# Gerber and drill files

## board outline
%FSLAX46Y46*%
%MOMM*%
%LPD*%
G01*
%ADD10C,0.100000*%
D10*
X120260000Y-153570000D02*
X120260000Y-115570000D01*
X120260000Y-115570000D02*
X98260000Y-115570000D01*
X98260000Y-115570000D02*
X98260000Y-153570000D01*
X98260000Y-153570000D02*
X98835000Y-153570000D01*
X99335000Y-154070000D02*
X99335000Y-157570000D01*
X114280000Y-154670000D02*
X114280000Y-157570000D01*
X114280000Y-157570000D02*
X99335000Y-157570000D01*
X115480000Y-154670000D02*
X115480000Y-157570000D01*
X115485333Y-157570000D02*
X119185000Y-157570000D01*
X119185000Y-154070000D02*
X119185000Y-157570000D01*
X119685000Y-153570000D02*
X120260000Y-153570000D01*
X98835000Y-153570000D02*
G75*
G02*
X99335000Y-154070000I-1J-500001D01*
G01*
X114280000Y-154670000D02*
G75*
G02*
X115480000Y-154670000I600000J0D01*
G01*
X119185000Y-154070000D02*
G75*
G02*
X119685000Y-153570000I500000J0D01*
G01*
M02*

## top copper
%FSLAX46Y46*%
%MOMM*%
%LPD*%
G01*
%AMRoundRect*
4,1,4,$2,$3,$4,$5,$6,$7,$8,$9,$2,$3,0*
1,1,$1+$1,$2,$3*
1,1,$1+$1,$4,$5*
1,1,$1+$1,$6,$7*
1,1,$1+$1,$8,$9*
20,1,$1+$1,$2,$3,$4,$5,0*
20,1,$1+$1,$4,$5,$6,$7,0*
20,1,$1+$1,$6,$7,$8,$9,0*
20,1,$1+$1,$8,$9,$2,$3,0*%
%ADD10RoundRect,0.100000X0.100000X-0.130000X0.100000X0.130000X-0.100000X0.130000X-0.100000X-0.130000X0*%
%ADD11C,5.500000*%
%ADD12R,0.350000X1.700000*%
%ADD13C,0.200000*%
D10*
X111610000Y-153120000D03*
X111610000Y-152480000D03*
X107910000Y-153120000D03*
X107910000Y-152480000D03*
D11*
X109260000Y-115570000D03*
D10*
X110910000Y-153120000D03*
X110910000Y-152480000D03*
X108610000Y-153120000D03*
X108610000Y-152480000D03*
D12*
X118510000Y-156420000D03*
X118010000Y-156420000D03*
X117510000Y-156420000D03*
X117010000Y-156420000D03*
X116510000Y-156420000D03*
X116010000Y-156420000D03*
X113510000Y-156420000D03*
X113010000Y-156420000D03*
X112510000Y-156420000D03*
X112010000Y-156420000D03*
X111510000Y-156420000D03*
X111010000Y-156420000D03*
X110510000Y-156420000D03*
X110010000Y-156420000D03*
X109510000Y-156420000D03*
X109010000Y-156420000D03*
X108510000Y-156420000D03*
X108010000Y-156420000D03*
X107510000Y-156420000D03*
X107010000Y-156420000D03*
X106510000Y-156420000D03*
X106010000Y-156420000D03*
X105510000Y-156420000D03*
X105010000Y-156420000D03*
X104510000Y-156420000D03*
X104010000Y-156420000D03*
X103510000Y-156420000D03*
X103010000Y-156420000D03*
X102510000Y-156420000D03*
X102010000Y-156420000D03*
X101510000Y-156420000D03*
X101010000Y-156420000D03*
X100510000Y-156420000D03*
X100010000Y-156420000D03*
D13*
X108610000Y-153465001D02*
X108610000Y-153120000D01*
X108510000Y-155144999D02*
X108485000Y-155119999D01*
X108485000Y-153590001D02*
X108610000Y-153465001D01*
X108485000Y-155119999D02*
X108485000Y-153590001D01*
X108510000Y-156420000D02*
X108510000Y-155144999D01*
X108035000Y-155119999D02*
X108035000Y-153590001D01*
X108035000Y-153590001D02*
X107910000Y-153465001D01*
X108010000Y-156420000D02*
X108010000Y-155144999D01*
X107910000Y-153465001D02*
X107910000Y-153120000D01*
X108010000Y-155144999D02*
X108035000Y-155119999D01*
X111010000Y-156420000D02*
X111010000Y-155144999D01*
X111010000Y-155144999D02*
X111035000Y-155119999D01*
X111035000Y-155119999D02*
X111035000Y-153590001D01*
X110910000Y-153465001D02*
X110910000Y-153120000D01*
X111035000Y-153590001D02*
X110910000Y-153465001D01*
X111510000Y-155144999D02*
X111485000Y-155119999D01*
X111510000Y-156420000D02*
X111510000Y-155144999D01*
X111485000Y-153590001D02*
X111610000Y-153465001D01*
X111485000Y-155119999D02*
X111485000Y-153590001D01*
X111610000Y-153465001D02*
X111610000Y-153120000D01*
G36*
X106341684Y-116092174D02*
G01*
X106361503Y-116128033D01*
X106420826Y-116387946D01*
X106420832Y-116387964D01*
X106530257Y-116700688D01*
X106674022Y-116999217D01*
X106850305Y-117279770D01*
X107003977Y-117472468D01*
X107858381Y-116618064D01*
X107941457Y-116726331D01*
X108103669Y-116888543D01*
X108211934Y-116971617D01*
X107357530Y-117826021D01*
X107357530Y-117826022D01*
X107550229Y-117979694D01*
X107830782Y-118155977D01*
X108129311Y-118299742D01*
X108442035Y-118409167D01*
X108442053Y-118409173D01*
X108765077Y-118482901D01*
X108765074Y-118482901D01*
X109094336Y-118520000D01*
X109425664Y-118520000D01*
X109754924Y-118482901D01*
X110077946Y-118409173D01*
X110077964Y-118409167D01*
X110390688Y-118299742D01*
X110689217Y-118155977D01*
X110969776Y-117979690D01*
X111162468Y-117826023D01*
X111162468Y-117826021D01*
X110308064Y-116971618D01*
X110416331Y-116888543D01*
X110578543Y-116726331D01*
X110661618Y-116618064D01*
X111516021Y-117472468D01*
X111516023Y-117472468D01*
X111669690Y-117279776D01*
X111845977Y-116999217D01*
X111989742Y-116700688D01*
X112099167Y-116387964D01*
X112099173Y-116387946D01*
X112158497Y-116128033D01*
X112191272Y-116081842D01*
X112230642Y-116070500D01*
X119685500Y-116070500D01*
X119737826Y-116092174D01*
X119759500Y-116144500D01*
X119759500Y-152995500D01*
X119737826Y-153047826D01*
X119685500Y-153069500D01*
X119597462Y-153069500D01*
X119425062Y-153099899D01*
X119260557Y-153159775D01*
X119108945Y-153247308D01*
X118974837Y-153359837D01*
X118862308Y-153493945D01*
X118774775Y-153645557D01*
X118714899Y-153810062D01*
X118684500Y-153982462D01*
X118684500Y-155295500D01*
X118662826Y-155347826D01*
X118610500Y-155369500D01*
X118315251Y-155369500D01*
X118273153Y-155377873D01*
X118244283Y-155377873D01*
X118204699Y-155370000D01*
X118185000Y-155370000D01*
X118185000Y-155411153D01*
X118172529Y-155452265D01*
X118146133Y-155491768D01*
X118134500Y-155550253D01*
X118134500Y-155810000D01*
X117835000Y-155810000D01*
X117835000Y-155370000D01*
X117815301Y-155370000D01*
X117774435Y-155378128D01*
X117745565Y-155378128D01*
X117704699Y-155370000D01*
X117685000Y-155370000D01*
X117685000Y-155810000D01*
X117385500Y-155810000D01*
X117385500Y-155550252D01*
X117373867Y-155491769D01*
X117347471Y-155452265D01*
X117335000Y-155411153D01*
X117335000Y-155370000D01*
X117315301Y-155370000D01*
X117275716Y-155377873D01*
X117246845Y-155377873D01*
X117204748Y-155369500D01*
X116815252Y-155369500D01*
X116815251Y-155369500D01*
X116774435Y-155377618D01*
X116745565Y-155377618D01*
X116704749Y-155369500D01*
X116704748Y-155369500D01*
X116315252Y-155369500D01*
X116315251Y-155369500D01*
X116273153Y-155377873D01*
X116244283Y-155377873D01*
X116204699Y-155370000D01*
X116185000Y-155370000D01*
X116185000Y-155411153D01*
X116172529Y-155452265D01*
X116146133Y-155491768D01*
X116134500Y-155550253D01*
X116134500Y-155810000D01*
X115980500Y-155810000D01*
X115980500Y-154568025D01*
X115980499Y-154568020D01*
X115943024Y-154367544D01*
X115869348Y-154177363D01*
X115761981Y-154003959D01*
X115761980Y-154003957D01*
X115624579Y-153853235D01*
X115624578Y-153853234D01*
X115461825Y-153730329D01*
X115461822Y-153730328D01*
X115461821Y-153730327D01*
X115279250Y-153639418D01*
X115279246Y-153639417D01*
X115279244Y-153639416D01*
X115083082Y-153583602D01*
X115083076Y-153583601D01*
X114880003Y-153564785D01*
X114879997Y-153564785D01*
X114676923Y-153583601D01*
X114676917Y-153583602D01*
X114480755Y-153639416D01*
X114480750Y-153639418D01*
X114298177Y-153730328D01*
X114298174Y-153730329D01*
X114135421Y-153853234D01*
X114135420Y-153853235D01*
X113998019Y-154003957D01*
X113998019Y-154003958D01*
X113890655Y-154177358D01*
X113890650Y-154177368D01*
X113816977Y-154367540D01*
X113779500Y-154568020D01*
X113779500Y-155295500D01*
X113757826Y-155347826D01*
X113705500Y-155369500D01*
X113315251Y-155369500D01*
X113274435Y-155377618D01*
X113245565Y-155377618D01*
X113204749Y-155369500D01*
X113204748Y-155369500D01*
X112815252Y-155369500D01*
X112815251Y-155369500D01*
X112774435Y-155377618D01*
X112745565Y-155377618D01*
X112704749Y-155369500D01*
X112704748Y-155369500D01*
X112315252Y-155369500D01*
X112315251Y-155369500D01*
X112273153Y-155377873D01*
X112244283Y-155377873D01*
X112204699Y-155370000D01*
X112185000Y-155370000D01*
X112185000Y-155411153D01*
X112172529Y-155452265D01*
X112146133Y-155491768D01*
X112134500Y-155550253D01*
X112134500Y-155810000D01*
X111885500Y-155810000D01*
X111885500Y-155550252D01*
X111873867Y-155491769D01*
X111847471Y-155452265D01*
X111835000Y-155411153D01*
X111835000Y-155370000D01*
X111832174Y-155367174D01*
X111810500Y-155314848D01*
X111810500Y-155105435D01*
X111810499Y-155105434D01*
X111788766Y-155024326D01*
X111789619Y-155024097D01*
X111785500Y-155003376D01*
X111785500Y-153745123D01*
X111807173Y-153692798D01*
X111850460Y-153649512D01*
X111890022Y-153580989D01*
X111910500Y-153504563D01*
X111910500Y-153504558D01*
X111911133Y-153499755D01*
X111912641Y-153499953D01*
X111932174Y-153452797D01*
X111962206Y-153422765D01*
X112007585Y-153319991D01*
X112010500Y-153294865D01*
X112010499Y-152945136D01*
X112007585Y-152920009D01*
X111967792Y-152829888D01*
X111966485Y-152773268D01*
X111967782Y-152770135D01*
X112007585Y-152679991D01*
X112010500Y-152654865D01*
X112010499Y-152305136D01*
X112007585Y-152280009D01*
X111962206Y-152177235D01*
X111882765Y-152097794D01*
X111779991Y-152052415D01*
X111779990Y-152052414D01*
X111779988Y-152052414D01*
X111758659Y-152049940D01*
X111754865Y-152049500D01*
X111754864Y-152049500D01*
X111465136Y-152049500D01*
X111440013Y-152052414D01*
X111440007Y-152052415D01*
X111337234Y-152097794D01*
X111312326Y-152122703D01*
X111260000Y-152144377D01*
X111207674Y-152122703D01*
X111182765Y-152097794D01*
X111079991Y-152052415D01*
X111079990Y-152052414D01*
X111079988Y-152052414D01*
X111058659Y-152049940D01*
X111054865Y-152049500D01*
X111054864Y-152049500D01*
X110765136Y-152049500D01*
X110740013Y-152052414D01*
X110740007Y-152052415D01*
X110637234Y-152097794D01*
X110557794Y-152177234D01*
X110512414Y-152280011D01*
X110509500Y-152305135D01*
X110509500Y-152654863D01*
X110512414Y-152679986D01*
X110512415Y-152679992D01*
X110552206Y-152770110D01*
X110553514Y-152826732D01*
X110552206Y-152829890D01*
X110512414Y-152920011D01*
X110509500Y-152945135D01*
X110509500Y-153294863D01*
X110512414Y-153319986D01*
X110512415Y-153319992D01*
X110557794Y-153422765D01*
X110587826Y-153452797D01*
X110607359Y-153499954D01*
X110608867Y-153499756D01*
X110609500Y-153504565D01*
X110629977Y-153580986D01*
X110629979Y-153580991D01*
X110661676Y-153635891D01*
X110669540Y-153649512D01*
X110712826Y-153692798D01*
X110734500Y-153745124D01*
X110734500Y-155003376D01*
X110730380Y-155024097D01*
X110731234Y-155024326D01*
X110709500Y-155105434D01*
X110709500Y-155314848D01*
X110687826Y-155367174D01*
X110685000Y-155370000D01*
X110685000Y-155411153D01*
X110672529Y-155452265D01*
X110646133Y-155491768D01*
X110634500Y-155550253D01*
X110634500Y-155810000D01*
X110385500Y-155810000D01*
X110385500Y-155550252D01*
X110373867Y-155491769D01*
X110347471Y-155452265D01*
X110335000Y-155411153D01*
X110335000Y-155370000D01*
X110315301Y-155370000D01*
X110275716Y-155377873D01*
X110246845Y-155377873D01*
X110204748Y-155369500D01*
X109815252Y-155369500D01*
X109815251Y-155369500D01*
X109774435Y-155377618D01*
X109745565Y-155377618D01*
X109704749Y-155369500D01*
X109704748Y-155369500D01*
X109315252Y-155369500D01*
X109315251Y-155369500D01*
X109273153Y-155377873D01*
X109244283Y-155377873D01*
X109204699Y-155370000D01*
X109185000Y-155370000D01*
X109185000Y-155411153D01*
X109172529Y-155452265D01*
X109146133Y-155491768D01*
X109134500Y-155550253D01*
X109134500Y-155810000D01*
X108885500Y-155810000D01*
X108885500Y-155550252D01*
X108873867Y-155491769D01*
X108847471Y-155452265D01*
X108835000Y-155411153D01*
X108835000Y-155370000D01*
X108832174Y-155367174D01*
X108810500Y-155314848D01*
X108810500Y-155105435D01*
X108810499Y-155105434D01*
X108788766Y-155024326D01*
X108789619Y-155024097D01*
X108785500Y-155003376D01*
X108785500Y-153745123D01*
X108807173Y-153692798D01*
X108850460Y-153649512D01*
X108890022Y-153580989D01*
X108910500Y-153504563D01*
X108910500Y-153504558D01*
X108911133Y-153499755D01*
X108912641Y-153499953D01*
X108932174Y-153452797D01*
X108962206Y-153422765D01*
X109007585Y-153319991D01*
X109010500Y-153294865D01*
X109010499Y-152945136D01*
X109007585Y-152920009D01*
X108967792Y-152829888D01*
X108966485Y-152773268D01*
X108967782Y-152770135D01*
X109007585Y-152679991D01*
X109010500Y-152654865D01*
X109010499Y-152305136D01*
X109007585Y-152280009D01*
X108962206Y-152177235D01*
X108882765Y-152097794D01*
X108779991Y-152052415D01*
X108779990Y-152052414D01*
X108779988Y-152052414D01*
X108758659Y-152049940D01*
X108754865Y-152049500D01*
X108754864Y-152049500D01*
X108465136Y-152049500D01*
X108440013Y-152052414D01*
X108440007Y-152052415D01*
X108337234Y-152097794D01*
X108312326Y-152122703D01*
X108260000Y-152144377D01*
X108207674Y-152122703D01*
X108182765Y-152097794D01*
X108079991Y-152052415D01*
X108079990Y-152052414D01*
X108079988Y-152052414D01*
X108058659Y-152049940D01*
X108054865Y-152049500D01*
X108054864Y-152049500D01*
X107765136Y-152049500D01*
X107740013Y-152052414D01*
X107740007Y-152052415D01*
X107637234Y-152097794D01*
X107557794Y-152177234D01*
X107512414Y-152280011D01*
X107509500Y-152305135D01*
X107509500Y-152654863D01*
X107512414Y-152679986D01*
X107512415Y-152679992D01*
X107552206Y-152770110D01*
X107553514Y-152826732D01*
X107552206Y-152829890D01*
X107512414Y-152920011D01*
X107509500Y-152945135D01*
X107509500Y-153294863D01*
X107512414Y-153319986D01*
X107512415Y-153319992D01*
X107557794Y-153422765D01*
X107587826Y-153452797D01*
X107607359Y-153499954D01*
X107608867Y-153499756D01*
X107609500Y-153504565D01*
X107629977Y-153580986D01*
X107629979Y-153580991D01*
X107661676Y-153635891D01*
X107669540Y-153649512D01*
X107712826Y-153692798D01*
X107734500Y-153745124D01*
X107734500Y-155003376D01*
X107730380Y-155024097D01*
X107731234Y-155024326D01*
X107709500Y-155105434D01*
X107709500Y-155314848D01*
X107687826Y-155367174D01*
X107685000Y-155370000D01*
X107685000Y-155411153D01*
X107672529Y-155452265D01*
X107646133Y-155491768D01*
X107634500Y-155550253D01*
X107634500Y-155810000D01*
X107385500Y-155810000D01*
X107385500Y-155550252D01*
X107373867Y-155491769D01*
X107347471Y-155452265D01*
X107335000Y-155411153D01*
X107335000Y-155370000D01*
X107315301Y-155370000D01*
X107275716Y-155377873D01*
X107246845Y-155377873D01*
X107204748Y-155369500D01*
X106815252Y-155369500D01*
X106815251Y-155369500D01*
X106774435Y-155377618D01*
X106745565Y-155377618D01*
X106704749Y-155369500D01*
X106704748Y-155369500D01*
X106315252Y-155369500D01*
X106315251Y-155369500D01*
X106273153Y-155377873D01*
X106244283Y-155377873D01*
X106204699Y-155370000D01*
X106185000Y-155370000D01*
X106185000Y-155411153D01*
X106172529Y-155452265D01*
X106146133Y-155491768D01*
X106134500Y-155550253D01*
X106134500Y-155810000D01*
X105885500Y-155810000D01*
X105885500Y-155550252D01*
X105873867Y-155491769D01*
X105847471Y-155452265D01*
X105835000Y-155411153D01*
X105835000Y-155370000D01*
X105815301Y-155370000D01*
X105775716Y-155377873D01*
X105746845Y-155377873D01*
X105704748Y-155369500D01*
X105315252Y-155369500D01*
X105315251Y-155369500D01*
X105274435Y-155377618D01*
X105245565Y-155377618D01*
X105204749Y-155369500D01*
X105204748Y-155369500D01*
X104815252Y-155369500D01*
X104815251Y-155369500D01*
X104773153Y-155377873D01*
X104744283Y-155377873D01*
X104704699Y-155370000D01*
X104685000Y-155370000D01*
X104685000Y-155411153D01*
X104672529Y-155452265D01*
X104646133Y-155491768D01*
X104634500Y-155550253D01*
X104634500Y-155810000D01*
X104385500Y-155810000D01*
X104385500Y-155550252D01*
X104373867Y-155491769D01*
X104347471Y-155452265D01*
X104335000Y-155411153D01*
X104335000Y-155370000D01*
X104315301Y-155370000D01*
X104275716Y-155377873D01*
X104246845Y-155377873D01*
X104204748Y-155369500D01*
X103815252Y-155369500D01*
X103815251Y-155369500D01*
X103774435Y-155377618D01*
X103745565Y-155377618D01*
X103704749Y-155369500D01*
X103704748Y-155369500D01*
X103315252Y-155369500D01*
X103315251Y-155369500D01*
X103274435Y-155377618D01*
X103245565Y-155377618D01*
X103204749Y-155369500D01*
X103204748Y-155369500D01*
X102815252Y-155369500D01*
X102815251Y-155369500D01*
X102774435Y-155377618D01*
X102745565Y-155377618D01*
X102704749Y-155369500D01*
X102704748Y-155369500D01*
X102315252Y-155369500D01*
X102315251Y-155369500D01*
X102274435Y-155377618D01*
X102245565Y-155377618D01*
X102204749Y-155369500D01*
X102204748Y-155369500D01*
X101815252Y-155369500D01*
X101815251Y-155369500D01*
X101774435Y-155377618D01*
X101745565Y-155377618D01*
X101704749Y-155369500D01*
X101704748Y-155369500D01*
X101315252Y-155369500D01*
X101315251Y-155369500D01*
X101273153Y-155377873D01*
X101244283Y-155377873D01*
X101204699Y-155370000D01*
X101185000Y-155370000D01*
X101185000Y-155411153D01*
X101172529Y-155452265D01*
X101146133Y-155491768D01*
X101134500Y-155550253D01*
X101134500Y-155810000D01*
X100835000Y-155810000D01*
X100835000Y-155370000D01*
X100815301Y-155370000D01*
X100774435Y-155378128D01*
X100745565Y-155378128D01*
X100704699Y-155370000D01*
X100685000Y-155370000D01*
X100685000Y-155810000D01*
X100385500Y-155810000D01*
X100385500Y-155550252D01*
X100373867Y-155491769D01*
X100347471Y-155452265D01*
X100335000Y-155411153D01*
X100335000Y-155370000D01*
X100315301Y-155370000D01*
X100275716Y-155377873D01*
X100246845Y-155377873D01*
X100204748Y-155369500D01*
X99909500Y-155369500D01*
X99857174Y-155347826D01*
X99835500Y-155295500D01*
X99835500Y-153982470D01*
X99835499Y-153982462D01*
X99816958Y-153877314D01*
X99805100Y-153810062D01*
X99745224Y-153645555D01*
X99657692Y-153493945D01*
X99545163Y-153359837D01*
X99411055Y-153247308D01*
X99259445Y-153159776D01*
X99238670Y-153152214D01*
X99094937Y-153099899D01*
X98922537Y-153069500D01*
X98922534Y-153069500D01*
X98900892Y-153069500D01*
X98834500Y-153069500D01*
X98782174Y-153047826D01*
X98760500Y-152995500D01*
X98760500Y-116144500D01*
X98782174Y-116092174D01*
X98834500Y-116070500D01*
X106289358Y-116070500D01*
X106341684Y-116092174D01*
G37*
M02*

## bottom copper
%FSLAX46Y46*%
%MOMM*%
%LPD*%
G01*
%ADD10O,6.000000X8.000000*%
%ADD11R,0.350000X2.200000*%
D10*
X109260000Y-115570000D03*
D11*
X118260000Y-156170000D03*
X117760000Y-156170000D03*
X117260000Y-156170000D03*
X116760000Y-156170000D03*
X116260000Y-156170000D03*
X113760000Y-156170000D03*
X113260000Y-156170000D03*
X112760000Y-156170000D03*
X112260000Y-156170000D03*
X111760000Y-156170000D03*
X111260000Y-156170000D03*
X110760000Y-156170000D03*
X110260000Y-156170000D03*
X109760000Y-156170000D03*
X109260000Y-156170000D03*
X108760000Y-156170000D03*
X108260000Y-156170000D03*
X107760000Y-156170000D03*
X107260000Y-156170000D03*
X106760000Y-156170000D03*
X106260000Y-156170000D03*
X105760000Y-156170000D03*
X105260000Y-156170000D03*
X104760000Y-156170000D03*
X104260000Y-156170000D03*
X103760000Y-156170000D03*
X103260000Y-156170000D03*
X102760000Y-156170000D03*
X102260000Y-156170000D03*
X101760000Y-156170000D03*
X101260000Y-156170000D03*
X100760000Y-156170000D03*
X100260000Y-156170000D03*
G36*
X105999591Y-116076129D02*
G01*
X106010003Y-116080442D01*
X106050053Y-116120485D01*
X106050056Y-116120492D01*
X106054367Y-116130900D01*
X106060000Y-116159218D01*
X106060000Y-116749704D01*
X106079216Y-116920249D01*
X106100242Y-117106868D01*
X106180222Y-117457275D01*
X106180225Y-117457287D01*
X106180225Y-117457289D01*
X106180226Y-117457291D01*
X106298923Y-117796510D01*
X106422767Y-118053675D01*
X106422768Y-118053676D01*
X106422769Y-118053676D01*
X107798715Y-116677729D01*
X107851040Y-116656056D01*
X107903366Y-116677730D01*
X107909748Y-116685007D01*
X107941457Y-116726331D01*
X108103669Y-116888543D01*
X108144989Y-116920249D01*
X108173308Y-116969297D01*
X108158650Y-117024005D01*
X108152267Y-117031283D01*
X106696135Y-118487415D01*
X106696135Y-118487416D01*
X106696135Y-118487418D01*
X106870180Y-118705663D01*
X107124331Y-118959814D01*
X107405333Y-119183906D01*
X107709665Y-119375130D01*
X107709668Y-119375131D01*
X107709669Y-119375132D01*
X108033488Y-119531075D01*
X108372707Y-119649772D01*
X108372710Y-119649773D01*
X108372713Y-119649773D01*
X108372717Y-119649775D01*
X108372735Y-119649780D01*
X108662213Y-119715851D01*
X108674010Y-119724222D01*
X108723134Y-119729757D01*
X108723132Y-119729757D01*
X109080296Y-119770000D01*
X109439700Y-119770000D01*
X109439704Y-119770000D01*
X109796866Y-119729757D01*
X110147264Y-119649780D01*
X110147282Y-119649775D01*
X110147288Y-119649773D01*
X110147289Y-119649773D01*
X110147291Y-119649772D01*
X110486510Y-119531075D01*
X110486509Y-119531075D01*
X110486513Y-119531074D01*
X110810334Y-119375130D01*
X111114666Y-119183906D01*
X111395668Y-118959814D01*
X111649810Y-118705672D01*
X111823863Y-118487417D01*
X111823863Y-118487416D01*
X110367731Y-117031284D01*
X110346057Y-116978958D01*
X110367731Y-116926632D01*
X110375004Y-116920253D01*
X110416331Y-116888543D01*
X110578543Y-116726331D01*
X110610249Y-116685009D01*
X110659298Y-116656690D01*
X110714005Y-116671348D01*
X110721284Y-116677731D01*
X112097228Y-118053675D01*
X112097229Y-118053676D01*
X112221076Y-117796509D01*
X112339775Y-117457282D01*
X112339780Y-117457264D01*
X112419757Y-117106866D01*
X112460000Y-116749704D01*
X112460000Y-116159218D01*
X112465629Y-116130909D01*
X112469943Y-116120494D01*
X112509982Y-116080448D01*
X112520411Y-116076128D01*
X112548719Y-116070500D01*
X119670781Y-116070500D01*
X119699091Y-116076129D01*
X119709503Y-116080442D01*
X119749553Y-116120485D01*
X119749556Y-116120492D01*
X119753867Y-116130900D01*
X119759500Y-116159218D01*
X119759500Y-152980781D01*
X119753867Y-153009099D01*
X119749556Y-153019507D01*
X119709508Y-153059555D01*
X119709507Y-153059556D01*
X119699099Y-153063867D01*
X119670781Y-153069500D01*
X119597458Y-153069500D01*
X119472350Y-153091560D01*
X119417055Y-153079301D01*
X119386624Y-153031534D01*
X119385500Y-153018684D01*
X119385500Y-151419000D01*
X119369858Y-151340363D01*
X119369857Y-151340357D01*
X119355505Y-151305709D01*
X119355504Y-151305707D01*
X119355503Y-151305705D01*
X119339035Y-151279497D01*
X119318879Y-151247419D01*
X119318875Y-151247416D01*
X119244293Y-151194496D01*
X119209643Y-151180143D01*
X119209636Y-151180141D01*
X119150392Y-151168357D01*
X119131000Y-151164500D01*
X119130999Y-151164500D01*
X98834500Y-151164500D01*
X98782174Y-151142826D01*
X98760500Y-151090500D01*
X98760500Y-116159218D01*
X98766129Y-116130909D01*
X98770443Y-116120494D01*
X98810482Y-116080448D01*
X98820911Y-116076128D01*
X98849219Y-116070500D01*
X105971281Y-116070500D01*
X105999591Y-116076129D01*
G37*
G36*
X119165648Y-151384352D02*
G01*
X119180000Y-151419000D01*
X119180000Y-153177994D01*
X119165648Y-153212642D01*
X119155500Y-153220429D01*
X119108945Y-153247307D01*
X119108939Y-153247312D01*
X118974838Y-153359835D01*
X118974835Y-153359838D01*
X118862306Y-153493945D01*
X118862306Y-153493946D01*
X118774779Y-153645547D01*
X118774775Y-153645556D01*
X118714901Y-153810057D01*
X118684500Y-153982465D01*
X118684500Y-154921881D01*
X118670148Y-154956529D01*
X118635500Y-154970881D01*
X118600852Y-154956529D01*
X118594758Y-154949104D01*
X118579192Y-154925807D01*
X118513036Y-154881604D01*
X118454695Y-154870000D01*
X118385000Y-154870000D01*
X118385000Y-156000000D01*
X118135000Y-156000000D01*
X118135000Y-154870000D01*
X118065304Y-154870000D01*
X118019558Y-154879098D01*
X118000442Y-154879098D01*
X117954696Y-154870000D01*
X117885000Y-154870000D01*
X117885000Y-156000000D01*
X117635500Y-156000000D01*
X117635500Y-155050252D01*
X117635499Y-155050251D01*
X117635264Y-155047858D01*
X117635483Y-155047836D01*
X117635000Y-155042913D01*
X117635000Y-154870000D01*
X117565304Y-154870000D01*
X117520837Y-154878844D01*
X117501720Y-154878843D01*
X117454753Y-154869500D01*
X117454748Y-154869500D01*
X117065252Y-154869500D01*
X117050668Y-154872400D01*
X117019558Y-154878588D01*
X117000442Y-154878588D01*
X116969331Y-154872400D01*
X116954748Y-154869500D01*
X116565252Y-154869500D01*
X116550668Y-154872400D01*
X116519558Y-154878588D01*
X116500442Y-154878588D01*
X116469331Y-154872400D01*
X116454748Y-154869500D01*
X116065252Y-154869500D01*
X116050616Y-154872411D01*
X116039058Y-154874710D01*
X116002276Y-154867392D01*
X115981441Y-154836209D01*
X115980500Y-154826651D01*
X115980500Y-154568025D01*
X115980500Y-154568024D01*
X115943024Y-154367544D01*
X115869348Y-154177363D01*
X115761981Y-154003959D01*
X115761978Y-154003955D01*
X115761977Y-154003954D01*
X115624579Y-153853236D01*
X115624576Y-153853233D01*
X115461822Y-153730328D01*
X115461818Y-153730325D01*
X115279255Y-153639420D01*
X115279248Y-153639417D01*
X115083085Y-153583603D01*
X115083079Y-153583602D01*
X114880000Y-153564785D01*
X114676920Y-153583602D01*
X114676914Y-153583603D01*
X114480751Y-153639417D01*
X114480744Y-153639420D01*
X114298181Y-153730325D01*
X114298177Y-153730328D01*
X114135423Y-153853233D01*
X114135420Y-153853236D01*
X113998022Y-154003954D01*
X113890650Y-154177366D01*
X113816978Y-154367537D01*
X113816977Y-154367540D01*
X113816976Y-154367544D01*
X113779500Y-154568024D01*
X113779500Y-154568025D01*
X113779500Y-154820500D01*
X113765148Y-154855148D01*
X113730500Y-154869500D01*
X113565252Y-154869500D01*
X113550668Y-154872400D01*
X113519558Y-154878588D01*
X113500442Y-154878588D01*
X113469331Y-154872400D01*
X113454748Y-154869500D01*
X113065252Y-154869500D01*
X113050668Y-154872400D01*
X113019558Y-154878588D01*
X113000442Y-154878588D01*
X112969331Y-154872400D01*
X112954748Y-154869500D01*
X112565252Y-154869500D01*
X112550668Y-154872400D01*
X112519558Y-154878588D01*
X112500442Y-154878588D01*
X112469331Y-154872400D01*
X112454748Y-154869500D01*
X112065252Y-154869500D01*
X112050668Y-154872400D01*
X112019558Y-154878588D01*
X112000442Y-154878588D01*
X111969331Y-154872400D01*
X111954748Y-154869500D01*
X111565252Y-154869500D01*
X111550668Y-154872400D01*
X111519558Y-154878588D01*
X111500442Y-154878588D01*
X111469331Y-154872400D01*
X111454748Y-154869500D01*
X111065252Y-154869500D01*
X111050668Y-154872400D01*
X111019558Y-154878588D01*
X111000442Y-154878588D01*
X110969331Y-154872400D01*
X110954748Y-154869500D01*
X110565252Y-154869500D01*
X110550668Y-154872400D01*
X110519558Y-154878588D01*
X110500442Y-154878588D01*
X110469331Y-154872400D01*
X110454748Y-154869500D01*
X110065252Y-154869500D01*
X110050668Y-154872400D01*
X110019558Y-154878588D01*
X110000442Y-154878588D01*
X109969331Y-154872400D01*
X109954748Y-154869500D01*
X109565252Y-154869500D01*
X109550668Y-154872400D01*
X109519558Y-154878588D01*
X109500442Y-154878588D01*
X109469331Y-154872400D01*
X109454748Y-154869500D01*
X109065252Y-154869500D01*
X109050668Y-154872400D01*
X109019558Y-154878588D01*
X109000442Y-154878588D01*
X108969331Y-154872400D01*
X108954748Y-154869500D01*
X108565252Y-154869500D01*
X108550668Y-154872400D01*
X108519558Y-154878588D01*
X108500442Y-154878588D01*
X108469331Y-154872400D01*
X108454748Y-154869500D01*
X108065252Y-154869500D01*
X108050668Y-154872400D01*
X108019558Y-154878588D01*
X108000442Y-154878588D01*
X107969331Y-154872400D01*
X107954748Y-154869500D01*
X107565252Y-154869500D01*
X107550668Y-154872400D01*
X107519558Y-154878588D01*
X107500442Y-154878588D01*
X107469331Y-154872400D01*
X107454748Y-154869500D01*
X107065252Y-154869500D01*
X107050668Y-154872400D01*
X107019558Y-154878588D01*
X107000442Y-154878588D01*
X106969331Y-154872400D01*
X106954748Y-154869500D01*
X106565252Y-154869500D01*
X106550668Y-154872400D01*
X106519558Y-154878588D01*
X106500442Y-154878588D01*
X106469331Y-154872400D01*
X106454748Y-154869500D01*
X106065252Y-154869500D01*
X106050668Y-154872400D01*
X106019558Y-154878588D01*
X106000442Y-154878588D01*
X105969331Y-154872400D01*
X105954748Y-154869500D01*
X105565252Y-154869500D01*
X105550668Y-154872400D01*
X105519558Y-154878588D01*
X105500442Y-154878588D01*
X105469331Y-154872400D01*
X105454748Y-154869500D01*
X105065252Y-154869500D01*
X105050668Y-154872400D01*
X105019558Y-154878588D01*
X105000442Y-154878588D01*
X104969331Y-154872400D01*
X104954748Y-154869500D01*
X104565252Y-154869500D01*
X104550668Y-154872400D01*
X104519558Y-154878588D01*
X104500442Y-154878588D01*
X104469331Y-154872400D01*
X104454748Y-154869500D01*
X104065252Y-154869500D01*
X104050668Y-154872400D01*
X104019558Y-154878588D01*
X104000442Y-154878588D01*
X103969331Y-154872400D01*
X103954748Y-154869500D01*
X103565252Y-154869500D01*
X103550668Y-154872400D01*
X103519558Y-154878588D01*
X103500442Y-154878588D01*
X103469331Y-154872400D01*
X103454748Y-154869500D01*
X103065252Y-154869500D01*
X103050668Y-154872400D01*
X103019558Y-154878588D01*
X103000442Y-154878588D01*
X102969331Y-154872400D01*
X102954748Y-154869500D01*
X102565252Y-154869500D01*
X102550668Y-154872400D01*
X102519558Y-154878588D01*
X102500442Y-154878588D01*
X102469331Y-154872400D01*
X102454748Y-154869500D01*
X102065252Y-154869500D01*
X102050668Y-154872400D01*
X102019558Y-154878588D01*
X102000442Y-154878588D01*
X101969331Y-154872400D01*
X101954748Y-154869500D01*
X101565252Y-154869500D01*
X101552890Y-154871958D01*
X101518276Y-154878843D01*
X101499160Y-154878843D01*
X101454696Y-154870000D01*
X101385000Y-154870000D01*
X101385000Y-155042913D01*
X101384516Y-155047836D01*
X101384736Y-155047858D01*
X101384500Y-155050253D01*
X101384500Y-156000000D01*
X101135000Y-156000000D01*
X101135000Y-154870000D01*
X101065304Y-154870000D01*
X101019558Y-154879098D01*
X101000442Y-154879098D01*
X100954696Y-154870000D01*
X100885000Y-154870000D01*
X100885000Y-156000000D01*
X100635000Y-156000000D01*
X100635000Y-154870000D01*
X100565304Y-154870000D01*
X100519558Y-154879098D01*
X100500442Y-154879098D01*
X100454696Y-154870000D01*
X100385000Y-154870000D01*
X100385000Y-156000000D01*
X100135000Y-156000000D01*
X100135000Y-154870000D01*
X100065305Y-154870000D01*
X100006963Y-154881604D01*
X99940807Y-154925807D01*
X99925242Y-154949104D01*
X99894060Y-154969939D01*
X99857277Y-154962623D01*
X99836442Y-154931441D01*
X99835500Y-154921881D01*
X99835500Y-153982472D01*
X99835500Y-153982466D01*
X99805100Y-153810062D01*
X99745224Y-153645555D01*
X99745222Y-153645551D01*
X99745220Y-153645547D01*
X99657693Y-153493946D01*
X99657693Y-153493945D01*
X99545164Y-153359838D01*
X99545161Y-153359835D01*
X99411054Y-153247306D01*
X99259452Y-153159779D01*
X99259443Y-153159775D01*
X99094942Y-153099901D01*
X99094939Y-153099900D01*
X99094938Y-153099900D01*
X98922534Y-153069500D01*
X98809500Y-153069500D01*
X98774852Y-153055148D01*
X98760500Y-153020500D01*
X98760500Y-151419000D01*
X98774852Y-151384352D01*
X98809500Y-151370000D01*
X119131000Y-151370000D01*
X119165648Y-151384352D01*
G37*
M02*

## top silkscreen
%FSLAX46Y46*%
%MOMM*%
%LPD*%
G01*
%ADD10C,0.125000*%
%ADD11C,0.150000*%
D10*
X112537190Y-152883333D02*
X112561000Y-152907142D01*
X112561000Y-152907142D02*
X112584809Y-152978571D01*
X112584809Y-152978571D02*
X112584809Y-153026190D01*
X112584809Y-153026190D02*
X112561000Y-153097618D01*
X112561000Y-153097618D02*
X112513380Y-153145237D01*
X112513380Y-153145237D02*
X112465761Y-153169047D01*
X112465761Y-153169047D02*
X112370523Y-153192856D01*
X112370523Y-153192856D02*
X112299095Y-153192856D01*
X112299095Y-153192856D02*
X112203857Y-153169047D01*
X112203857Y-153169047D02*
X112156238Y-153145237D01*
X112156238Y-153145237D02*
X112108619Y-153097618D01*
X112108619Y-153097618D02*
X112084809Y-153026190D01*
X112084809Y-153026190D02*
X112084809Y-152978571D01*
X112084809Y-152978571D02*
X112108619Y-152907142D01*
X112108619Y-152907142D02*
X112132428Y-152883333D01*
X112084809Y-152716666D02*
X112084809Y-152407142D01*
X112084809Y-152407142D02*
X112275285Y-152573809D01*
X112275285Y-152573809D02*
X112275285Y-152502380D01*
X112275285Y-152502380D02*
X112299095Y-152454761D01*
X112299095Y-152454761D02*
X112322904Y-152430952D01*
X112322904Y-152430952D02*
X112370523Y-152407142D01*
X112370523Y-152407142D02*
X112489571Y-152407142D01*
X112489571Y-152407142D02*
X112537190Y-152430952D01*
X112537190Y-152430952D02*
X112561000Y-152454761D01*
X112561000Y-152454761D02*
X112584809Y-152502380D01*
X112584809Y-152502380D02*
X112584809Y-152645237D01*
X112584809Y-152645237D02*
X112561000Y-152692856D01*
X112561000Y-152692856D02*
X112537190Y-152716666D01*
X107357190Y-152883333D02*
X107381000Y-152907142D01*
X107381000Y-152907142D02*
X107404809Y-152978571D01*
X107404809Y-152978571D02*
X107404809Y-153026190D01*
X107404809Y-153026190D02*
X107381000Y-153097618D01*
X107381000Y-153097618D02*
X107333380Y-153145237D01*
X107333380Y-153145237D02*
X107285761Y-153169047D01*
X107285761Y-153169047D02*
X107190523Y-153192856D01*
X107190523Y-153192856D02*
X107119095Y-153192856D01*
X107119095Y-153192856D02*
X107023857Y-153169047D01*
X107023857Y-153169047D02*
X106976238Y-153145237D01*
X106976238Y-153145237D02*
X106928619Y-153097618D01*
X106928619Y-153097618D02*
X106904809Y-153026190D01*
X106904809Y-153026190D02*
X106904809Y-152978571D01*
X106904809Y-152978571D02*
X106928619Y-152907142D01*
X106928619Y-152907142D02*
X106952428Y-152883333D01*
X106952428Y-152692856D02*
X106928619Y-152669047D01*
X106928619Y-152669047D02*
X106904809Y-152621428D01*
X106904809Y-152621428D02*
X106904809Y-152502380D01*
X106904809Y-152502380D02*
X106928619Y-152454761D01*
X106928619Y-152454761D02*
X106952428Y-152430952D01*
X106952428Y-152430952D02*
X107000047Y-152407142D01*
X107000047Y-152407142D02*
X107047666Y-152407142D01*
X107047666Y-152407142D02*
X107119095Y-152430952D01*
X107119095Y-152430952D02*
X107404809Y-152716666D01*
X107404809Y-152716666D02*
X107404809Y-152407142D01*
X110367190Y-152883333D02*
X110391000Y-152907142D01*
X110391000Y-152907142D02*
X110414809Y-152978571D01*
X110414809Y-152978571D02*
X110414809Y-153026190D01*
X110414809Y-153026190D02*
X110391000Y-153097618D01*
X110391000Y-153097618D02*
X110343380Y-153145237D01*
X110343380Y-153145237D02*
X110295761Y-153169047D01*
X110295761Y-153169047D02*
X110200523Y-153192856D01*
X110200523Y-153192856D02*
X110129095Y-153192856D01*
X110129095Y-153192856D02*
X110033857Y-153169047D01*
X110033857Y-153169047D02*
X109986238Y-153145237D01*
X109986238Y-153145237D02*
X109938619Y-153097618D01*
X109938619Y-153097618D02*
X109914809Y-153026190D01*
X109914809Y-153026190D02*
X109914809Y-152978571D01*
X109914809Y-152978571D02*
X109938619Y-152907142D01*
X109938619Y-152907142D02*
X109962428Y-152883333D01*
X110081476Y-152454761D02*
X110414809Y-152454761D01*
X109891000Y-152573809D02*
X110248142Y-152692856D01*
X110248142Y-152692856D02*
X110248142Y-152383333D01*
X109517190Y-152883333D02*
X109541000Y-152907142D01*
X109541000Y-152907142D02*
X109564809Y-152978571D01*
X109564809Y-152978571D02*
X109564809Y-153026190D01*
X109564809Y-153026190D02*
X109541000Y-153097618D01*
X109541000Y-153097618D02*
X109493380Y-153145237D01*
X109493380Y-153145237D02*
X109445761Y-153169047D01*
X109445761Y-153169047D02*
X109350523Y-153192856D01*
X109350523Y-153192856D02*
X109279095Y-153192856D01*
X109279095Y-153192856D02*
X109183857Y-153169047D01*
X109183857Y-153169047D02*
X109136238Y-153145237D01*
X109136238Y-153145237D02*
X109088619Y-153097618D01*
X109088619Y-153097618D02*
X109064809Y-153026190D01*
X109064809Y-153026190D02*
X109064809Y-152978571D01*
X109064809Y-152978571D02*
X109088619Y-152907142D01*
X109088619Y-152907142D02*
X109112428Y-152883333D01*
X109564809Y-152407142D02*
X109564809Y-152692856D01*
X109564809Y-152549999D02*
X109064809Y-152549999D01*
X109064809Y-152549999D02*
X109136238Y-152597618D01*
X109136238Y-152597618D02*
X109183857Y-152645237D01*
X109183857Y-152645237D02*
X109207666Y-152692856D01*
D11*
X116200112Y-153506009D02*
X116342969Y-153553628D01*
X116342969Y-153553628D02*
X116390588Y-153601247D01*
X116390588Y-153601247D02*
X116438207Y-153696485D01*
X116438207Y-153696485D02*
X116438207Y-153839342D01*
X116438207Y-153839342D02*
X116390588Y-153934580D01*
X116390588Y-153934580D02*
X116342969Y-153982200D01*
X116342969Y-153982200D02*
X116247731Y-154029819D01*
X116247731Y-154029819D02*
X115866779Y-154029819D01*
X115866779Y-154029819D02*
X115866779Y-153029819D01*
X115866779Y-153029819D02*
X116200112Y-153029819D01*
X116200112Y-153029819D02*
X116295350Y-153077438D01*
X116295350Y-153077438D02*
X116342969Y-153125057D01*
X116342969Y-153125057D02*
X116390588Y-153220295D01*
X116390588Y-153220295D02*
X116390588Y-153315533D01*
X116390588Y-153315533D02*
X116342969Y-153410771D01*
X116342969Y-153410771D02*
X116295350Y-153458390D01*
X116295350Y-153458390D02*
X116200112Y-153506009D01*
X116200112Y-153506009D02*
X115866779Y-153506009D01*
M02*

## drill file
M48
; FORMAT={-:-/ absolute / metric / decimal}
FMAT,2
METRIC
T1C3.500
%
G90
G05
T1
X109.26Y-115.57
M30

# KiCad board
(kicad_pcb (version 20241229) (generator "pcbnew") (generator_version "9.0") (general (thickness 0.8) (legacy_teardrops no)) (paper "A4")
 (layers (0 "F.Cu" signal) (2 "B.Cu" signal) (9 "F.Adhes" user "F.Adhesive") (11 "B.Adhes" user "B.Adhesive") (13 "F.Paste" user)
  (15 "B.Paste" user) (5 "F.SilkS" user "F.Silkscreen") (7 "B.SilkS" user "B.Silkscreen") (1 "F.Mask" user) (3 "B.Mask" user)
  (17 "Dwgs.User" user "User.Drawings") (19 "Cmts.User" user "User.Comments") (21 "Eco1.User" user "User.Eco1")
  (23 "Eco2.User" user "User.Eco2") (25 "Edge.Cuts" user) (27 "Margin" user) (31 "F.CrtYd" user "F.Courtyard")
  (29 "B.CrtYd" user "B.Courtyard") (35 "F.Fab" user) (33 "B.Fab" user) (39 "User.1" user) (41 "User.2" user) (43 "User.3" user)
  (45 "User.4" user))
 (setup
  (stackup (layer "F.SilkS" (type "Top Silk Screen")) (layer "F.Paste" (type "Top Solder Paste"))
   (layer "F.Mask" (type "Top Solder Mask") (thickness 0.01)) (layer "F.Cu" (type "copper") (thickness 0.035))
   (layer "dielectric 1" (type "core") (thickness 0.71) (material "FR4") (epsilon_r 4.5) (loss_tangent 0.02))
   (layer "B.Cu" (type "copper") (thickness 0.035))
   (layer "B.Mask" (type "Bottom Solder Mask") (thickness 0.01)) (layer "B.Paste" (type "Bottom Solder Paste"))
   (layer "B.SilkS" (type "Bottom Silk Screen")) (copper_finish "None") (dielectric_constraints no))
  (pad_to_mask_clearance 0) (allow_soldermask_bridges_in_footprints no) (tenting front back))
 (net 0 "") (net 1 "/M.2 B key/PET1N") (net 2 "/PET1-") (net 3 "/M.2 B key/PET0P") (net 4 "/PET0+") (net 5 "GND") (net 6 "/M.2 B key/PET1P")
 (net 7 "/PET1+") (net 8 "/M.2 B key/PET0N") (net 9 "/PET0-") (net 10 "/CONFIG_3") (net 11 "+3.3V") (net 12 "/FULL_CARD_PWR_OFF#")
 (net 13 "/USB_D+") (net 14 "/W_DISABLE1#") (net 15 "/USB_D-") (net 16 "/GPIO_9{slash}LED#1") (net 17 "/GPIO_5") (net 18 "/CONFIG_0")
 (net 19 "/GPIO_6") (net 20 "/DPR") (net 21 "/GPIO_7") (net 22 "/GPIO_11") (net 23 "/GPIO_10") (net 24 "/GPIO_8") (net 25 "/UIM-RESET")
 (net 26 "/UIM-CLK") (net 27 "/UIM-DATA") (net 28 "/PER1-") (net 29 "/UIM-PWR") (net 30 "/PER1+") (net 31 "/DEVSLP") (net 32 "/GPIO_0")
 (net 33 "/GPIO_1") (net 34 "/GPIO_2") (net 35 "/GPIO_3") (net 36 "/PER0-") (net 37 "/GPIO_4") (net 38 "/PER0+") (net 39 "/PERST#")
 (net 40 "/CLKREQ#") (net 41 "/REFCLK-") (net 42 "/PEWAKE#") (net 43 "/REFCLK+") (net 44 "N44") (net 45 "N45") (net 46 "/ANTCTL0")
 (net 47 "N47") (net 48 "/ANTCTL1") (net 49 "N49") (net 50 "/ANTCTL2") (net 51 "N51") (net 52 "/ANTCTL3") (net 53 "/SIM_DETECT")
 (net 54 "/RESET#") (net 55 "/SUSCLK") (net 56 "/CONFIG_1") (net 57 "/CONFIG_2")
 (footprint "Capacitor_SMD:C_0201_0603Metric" (layer "F.Cu") (at 111.61 152.8 90)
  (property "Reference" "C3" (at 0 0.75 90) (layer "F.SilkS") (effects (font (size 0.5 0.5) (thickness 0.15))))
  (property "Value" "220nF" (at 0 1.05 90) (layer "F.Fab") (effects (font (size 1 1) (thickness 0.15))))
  (pad "" smd roundrect (at -0.345 0 90) (size 0.318 0.36) (layers "F.Paste") (roundrect_rratio 0.25))
  (pad "" smd roundrect (at 0.345 0 90) (size 0.318 0.36) (layers "F.Paste") (roundrect_rratio 0.25))
  (pad "1" smd roundrect (at -0.32 0 90) (size 0.46 0.4) (layers "F.Cu" "F.Mask") (roundrect_rratio 0.25) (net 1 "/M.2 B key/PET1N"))
  (pad "2" smd roundrect (at 0.32 0 90) (size 0.46 0.4) (layers "F.Cu" "F.Mask") (roundrect_rratio 0.25) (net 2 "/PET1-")))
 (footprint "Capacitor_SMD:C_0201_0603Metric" (layer "F.Cu") (at 107.91 152.8 90)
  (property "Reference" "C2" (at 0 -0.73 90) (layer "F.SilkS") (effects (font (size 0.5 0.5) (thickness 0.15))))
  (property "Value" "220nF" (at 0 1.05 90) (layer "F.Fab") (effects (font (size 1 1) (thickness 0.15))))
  (pad "" smd roundrect (at -0.345 0 90) (size 0.318 0.36) (layers "F.Paste") (roundrect_rratio 0.25))
  (pad "" smd roundrect (at 0.345 0 90) (size 0.318 0.36) (layers "F.Paste") (roundrect_rratio 0.25))
  (pad "1" smd roundrect (at -0.32 0 90) (size 0.46 0.4) (layers "F.Cu" "F.Mask") (roundrect_rratio 0.25) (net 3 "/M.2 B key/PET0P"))
  (pad "2" smd roundrect (at 0.32 0 90) (size 0.46 0.4) (layers "F.Cu" "F.Mask") (roundrect_rratio 0.25) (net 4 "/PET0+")))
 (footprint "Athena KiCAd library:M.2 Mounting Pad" (layer "F.Cu") (at 109.26 115.57)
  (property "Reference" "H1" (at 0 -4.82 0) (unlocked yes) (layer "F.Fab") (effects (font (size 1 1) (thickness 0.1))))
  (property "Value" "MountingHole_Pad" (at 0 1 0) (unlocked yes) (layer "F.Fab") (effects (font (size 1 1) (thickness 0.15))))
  (pad "1" thru_hole circle (at 0 0) (size 5.5 5.5) (drill 3.5) (layers "*.Cu" "*.Mask") (remove_unused_layers no) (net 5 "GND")
   (padstack (mode front_inner_back)
    (layer "Inner" (shape circle) (size 5.5 5.5) (zone_connect -1))
    (layer "B.Cu" (shape oval) (size 6 8) (thermal_bridge_angle 45) (zone_connect -1)))))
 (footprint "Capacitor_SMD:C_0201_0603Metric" (layer "F.Cu") (at 110.91 152.8 90)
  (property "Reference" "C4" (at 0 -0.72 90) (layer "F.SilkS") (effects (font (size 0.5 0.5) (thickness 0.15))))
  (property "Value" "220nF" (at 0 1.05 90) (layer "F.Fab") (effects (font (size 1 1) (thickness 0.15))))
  (pad "" smd roundrect (at -0.345 0 90) (size 0.318 0.36) (layers "F.Paste") (roundrect_rratio 0.25))
  (pad "" smd roundrect (at 0.345 0 90) (size 0.318 0.36) (layers "F.Paste") (roundrect_rratio 0.25))
  (pad "1" smd roundrect (at -0.32 0 90) (size 0.46 0.4) (layers "F.Cu" "F.Mask") (roundrect_rratio 0.25) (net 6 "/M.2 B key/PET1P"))
  (pad "2" smd roundrect (at 0.32 0 90) (size 0.46 0.4) (layers "F.Cu" "F.Mask") (roundrect_rratio 0.25) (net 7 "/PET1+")))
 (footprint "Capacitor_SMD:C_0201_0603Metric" (layer "F.Cu") (at 108.61 152.8 90)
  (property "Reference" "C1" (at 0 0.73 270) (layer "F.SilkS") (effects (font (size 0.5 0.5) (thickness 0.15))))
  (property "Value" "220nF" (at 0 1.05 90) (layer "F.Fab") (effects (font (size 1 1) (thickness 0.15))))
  (pad "" smd roundrect (at -0.345 0 90) (size 0.318 0.36) (layers "F.Paste") (roundrect_rratio 0.25))
  (pad "" smd roundrect (at 0.345 0 90) (size 0.318 0.36) (layers "F.Paste") (roundrect_rratio 0.25))
  (pad "1" smd roundrect (at -0.32 0 90) (size 0.46 0.4) (layers "F.Cu" "F.Mask") (roundrect_rratio 0.25) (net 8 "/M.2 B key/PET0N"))
  (pad "2" smd roundrect (at 0.32 0 90) (size 0.46 0.4) (layers "F.Cu" "F.Mask") (roundrect_rratio 0.25) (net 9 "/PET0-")))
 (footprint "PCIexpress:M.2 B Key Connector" (layer "F.Cu") (at 109.26 156.46)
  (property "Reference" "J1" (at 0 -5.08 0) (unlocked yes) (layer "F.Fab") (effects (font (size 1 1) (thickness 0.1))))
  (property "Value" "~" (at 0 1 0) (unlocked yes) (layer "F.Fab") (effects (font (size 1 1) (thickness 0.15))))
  (fp_line (start -11 -2.89) (end -10.425 -2.89) (stroke (width 0.1) (type default)) (layer "Edge.Cuts"))
  (fp_line (start -9.925 -2.39) (end -9.925 1.11) (stroke (width 0.1) (type default)) (layer "Edge.Cuts"))
  (fp_line (start 5.02 -1.79) (end 5.02 1.11) (stroke (width 0.1) (type default)) (layer "Edge.Cuts"))
  (fp_line (start 5.02 1.11) (end -9.925 1.11) (stroke (width 0.1) (type default)) (layer "Edge.Cuts"))
  (fp_line (start 6.22 -1.79) (end 6.22 1.11) (stroke (width 0.1) (type default)) (layer "Edge.Cuts"))
  (fp_line (start 6.225333 1.11) (end 9.925 1.11) (stroke (width 0.1) (type default)) (layer "Edge.Cuts"))
  (fp_line (start 9.925 -2.39) (end 9.925 1.11) (stroke (width 0.1) (type default)) (layer "Edge.Cuts"))
  (fp_line (start 10.425 -2.89) (end 11 -2.89) (stroke (width 0.1) (type default)) (layer "Edge.Cuts"))
  (fp_arc (start -10.425 -2.89) (mid -10.071447 -2.743553) (end -9.925 -2.39) (stroke (width 0.1) (type default)) (layer "Edge.Cuts"))
  (fp_arc (start 5.02 -1.79) (mid 5.62 -2.39) (end 6.22 -1.79) (stroke (width 0.1) (type default)) (layer "Edge.Cuts"))
  (fp_arc (start 9.925 -2.39) (mid 10.071447 -2.743553) (end 10.425 -2.89) (stroke (width 0.1) (type default)) (layer "Edge.Cuts"))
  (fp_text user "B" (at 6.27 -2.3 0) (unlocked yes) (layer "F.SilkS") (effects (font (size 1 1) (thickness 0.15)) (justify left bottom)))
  (pad "1" smd rect (at 9.25 -0.04 180) (size 0.35 1.7) (layers "F.Cu") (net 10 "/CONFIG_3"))
  (pad "2" smd rect (at 9 -0.29 180) (size 0.35 2.2) (layers "B.Cu") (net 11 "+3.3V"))
  (pad "3" smd rect (at 8.75 -0.04 180) (size 0.35 1.7) (layers "F.Cu") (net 5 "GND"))
  (pad "4" smd rect (at 8.5 -0.29 180) (size 0.35 2.2) (layers "B.Cu") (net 11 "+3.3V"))
  (pad "5" smd rect (at 8.25 -0.04 180) (size 0.35 1.7) (layers "F.Cu") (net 5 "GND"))
  (pad "6" smd rect (at 8 -0.29 180) (size 0.35 2.2) (layers "B.Cu") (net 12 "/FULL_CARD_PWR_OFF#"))
  (pad "7" smd rect (at 7.75 -0.04 180) (size 0.35 1.7) (layers "F.Cu") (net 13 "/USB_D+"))
  (pad "8" smd rect (at 7.5 -0.29 180) (size 0.35 2.2) (layers "B.Cu") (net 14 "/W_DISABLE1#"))
  (pad "9" smd rect (at 7.25 -0.04 180) (size 0.35 1.7) (layers "F.Cu") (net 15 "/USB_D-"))
  (pad "10" smd rect (at 7 -0.29 180) (size 0.35 2.2) (layers "B.Cu") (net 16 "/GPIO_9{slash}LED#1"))
  (pad "11" smd rect (at 6.75 -0.04 180) (size 0.35 1.7) (layers "F.Cu") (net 5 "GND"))
  (pad "20" smd rect (at 4.5 -0.29 180) (size 0.35 2.2) (layers "B.Cu") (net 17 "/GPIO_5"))
  (pad "21" smd rect (at 4.25 -0.04 180) (size 0.35 1.7) (layers "F.Cu") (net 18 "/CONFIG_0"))
  (pad "22" smd rect (at 4 -0.29 180) (size 0.35 2.2) (layers "B.Cu") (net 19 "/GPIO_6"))
  (pad "23" smd rect (at 3.75 -0.04 180) (size 0.35 1.7) (layers "F.Cu") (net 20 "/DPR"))
  (pad "24" smd rect (at 3.5 -0.29 180) (size 0.35 2.2) (layers "B.Cu") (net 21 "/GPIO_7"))
  (pad "25" smd rect (at 3.25 -0.04 180) (size 0.35 1.7) (layers "F.Cu") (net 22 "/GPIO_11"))
  (pad "26" smd rect (at 3 -0.29 180) (size 0.35 2.2) (layers "B.Cu") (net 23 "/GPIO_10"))
  (pad "27" smd rect (at 2.75 -0.04 180) (size 0.35 1.7) (layers "F.Cu") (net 5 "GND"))
  (pad "28" smd rect (at 2.5 -0.29 180) (size 0.35 2.2) (layers "B.Cu") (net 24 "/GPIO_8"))
  (pad "29" smd rect (at 2.25 -0.04 180) (size 0.35 1.7) (layers "F.Cu") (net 1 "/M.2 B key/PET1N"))
  (pad "30" smd rect (at 2 -0.29 180) (size 0.35 2.2) (layers "B.Cu") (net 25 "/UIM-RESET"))
  (pad "31" smd rect (at 1.75 -0.04 180) (size 0.35 1.7) (layers "F.Cu") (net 6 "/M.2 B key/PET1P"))
  (pad "32" smd rect (at 1.5 -0.29 180) (size 0.35 2.2) (layers "B.Cu") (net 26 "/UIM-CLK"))
  (pad "33" smd rect (at 1.25 -0.04 180) (size 0.35 1.7) (layers "F.Cu") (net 5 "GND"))
  (pad "34" smd rect (at 1 -0.29 180) (size 0.35 2.2) (layers "B.Cu") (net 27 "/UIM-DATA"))
  (pad "35" smd rect (at 0.75 -0.04 180) (size 0.35 1.7) (layers "F.Cu") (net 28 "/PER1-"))
  (pad "36" smd rect (at 0.5 -0.29 180) (size 0.35 2.2) (layers "B.Cu") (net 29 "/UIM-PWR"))
  (pad "37" smd rect (at 0.25 -0.04 180) (size 0.35 1.7) (layers "F.Cu") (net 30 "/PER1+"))
  (pad "38" smd rect (at 0 -0.29 180) (size 0.35 2.2) (layers "B.Cu") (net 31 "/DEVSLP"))
  (pad "39" smd rect (at -0.25 -0.04 180) (size 0.35 1.7) (layers "F.Cu") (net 5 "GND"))
  (pad "40" smd rect (at -0.5 -0.29 180) (size 0.35 2.2) (layers "B.Cu") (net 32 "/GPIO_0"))
  (pad "41" smd rect (at -0.75 -0.04 180) (size 0.35 1.7) (layers "F.Cu") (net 8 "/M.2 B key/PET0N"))
  (pad "42" smd rect (at -1 -0.29 180) (size 0.35 2.2) (layers "B.Cu") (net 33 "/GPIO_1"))
  (pad "43" smd rect (at -1.25 -0.04 180) (size 0.35 1.7) (layers "F.Cu") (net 3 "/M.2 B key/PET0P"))
  (pad "44" smd rect (at -1.5 -0.29 180) (size 0.35 2.2) (layers "B.Cu") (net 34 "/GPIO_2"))
  (pad "45" smd rect (at -1.75 -0.04 180) (size 0.35 1.7) (layers "F.Cu") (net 5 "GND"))
  (pad "46" smd rect (at -2 -0.29 180) (size 0.35 2.2) (layers "B.Cu") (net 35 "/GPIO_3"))
  (pad "47" smd rect (at -2.25 -0.04 180) (size 0.35 1.7) (layers "F.Cu") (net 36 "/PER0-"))
  (pad "48" smd rect (at -2.5 -0.29 180) (size 0.35 2.2) (layers "B.Cu") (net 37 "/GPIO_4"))
  (pad "49" smd rect (at -2.75 -0.04 180) (size 0.35 1.7) (layers "F.Cu") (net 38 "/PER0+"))
  (pad "50" smd rect (at -3 -0.29 180) (size 0.35 2.2) (layers "B.Cu") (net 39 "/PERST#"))
  (pad "51" smd rect (at -3.25 -0.04 180) (size 0.35 1.7) (layers "F.Cu") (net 5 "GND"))
  (pad "52" smd rect (at -3.5 -0.29 180) (size 0.35 2.2) (layers "B.Cu") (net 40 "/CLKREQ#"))
  (pad "53" smd rect (at -3.75 -0.04 180) (size 0.35 1.7) (layers "F.Cu") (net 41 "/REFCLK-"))
  (pad "54" smd rect (at -4 -0.29 180) (size 0.35 2.2) (layers "B.Cu") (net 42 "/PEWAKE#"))
  (pad "55" smd rect (at -4.25 -0.04 180) (size 0.35 1.7) (layers "F.Cu") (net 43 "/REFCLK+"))
  (pad "56" smd rect (at -4.5 -0.29 180) (size 0.35 2.2) (layers "B.Cu") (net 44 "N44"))
  (pad "57" smd rect (at -4.75 -0.04 180) (size 0.35 1.7) (layers "F.Cu") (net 5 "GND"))
  (pad "58" smd rect (at -5 -0.29 180) (size 0.35 2.2) (layers "B.Cu") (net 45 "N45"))
  (pad "59" smd rect (at -5.25 -0.04 180) (size 0.35 1.7) (layers "F.Cu") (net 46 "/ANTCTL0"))
  (pad "60" smd rect (at -5.5 -0.29 180) (size 0.35 2.2) (layers "B.Cu") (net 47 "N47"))
  (pad "61" smd rect (at -5.75 -0.04 180) (size 0.35 1.7) (layers "F.Cu") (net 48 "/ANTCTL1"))
  (pad "62" smd rect (at -6 -0.29 180) (size 0.35 2.2) (layers "B.Cu") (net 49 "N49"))
  (pad "63" smd rect (at -6.25 -0.04 180) (size 0.35 1.7) (layers "F.Cu") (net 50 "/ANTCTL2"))
  (pad "64" smd rect (at -6.5 -0.29 180) (size 0.35 2.2) (layers "B.Cu") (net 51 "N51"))
  (pad "65" smd rect (at -6.75 -0.04 180) (size 0.35 1.7) (layers "F.Cu") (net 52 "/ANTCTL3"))
  (pad "66" smd rect (at -7 -0.29 180) (size 0.35 2.2) (layers "B.Cu") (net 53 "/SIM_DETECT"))
  (pad "67" smd rect (at -7.25 -0.04 180) (size 0.35 1.7) (layers "F.Cu") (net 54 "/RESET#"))
  (pad "68" smd rect (at -7.5 -0.29 180) (size 0.35 2.2) (layers "B.Cu") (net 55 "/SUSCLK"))
  (pad "69" smd rect (at -7.75 -0.04 180) (size 0.35 1.7) (layers "F.Cu") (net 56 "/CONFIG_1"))
  (pad "70" smd rect (at -8 -0.29 180) (size 0.35 2.2) (layers "B.Cu") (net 11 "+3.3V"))
  (pad "71" smd rect (at -8.25 -0.04 180) (size 0.35 1.7) (layers "F.Cu") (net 5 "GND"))
  (pad "72" smd rect (at -8.5 -0.29 180) (size 0.35 2.2) (layers "B.Cu") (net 11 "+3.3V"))
  (pad "73" smd rect (at -8.75 -0.04 180) (size 0.35 1.7) (layers "F.Cu") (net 5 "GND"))
  (pad "74" smd rect (at -9 -0.29 180) (size 0.35 2.2) (layers "B.Cu") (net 11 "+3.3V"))
  (pad "75" smd rect (at -9.25 -0.04 180) (size 0.35 1.7) (layers "F.Cu") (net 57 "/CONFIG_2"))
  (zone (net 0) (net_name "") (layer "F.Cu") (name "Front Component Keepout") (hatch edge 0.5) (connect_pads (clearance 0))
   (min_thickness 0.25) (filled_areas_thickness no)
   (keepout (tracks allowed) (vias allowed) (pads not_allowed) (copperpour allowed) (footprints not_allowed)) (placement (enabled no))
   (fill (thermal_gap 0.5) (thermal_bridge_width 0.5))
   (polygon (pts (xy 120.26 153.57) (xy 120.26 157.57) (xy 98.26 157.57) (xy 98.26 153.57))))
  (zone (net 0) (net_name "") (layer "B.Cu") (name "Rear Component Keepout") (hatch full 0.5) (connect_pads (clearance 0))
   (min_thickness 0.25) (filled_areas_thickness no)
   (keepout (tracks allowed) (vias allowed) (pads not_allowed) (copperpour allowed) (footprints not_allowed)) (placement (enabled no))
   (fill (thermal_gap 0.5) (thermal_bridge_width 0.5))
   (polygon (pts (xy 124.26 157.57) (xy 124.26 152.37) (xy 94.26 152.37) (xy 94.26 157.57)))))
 (gr_line (start 120.26 153.57) (end 120.26 115.57) (stroke (width 0.1) (type default)) (layer "Edge.Cuts"))
 (gr_line (start 120.26 115.57) (end 98.26 115.57) (stroke (width 0.1) (type default)) (layer "Edge.Cuts"))
 (gr_line (start 98.26 115.57) (end 98.26 153.57) (stroke (width 0.1) (type default)) (layer "Edge.Cuts"))
 (segment (start 108.61 153.465001) (end 108.61 153.12) (width 0.2) (layer "F.Cu") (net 8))
 (segment (start 108.51 155.144999) (end 108.485 155.119999) (width 0.2) (layer "F.Cu") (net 8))
 (segment (start 108.485 153.590001) (end 108.61 153.465001) (width 0.2) (layer "F.Cu") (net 8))
 (segment (start 108.485 155.119999) (end 108.485 153.590001) (width 0.2) (layer "F.Cu") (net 8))
 (segment (start 108.51 156.42) (end 108.51 155.144999) (width 0.2) (layer "F.Cu") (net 8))
 (segment (start 108.035 155.119999) (end 108.035 153.590001) (width 0.2) (layer "F.Cu") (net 3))
 (segment (start 108.035 153.590001) (end 107.91 153.465001) (width 0.2) (layer "F.Cu") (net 3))
 (segment (start 108.01 156.42) (end 108.01 155.144999) (width 0.2) (layer "F.Cu") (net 3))
 (segment (start 107.91 153.465001) (end 107.91 153.12) (width 0.2) (layer "F.Cu") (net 3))
 (segment (start 108.01 155.144999) (end 108.035 155.119999) (width 0.2) (layer "F.Cu") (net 3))
 (segment (start 111.01 156.42) (end 111.01 155.144999) (width 0.2) (layer "F.Cu") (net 6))
 (segment (start 111.01 155.144999) (end 111.035 155.119999) (width 0.2) (layer "F.Cu") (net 6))
 (segment (start 111.035 155.119999) (end 111.035 153.590001) (width 0.2) (layer "F.Cu") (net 6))
 (segment (start 110.91 153.465001) (end 110.91 153.12) (width 0.2) (layer "F.Cu") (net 6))
 (segment (start 111.035 153.590001) (end 110.91 153.465001) (width 0.2) (layer "F.Cu") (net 6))
 (segment (start 111.51 155.144999) (end 111.485 155.119999) (width 0.2) (layer "F.Cu") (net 1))
 (segment (start 111.51 156.42) (end 111.51 155.144999) (width 0.2) (layer "F.Cu") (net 1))
 (segment (start 111.485 153.590001) (end 111.61 153.465001) (width 0.2) (layer "F.Cu") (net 1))
 (segment (start 111.485 155.119999) (end 111.485 153.590001) (width 0.2) (layer "F.Cu") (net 1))
 (segment (start 111.61 153.465001) (end 111.61 153.12) (width 0.2) (layer "F.Cu") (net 1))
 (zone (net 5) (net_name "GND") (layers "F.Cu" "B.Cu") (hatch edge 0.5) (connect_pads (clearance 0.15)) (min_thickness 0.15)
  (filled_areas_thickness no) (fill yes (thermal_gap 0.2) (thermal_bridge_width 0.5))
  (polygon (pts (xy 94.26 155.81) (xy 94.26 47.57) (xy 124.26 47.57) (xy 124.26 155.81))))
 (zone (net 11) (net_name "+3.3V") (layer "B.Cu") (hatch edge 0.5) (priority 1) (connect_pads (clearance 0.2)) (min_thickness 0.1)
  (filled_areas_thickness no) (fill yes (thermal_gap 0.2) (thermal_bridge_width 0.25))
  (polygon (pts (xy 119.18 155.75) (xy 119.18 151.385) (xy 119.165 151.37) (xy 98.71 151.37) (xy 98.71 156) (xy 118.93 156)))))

